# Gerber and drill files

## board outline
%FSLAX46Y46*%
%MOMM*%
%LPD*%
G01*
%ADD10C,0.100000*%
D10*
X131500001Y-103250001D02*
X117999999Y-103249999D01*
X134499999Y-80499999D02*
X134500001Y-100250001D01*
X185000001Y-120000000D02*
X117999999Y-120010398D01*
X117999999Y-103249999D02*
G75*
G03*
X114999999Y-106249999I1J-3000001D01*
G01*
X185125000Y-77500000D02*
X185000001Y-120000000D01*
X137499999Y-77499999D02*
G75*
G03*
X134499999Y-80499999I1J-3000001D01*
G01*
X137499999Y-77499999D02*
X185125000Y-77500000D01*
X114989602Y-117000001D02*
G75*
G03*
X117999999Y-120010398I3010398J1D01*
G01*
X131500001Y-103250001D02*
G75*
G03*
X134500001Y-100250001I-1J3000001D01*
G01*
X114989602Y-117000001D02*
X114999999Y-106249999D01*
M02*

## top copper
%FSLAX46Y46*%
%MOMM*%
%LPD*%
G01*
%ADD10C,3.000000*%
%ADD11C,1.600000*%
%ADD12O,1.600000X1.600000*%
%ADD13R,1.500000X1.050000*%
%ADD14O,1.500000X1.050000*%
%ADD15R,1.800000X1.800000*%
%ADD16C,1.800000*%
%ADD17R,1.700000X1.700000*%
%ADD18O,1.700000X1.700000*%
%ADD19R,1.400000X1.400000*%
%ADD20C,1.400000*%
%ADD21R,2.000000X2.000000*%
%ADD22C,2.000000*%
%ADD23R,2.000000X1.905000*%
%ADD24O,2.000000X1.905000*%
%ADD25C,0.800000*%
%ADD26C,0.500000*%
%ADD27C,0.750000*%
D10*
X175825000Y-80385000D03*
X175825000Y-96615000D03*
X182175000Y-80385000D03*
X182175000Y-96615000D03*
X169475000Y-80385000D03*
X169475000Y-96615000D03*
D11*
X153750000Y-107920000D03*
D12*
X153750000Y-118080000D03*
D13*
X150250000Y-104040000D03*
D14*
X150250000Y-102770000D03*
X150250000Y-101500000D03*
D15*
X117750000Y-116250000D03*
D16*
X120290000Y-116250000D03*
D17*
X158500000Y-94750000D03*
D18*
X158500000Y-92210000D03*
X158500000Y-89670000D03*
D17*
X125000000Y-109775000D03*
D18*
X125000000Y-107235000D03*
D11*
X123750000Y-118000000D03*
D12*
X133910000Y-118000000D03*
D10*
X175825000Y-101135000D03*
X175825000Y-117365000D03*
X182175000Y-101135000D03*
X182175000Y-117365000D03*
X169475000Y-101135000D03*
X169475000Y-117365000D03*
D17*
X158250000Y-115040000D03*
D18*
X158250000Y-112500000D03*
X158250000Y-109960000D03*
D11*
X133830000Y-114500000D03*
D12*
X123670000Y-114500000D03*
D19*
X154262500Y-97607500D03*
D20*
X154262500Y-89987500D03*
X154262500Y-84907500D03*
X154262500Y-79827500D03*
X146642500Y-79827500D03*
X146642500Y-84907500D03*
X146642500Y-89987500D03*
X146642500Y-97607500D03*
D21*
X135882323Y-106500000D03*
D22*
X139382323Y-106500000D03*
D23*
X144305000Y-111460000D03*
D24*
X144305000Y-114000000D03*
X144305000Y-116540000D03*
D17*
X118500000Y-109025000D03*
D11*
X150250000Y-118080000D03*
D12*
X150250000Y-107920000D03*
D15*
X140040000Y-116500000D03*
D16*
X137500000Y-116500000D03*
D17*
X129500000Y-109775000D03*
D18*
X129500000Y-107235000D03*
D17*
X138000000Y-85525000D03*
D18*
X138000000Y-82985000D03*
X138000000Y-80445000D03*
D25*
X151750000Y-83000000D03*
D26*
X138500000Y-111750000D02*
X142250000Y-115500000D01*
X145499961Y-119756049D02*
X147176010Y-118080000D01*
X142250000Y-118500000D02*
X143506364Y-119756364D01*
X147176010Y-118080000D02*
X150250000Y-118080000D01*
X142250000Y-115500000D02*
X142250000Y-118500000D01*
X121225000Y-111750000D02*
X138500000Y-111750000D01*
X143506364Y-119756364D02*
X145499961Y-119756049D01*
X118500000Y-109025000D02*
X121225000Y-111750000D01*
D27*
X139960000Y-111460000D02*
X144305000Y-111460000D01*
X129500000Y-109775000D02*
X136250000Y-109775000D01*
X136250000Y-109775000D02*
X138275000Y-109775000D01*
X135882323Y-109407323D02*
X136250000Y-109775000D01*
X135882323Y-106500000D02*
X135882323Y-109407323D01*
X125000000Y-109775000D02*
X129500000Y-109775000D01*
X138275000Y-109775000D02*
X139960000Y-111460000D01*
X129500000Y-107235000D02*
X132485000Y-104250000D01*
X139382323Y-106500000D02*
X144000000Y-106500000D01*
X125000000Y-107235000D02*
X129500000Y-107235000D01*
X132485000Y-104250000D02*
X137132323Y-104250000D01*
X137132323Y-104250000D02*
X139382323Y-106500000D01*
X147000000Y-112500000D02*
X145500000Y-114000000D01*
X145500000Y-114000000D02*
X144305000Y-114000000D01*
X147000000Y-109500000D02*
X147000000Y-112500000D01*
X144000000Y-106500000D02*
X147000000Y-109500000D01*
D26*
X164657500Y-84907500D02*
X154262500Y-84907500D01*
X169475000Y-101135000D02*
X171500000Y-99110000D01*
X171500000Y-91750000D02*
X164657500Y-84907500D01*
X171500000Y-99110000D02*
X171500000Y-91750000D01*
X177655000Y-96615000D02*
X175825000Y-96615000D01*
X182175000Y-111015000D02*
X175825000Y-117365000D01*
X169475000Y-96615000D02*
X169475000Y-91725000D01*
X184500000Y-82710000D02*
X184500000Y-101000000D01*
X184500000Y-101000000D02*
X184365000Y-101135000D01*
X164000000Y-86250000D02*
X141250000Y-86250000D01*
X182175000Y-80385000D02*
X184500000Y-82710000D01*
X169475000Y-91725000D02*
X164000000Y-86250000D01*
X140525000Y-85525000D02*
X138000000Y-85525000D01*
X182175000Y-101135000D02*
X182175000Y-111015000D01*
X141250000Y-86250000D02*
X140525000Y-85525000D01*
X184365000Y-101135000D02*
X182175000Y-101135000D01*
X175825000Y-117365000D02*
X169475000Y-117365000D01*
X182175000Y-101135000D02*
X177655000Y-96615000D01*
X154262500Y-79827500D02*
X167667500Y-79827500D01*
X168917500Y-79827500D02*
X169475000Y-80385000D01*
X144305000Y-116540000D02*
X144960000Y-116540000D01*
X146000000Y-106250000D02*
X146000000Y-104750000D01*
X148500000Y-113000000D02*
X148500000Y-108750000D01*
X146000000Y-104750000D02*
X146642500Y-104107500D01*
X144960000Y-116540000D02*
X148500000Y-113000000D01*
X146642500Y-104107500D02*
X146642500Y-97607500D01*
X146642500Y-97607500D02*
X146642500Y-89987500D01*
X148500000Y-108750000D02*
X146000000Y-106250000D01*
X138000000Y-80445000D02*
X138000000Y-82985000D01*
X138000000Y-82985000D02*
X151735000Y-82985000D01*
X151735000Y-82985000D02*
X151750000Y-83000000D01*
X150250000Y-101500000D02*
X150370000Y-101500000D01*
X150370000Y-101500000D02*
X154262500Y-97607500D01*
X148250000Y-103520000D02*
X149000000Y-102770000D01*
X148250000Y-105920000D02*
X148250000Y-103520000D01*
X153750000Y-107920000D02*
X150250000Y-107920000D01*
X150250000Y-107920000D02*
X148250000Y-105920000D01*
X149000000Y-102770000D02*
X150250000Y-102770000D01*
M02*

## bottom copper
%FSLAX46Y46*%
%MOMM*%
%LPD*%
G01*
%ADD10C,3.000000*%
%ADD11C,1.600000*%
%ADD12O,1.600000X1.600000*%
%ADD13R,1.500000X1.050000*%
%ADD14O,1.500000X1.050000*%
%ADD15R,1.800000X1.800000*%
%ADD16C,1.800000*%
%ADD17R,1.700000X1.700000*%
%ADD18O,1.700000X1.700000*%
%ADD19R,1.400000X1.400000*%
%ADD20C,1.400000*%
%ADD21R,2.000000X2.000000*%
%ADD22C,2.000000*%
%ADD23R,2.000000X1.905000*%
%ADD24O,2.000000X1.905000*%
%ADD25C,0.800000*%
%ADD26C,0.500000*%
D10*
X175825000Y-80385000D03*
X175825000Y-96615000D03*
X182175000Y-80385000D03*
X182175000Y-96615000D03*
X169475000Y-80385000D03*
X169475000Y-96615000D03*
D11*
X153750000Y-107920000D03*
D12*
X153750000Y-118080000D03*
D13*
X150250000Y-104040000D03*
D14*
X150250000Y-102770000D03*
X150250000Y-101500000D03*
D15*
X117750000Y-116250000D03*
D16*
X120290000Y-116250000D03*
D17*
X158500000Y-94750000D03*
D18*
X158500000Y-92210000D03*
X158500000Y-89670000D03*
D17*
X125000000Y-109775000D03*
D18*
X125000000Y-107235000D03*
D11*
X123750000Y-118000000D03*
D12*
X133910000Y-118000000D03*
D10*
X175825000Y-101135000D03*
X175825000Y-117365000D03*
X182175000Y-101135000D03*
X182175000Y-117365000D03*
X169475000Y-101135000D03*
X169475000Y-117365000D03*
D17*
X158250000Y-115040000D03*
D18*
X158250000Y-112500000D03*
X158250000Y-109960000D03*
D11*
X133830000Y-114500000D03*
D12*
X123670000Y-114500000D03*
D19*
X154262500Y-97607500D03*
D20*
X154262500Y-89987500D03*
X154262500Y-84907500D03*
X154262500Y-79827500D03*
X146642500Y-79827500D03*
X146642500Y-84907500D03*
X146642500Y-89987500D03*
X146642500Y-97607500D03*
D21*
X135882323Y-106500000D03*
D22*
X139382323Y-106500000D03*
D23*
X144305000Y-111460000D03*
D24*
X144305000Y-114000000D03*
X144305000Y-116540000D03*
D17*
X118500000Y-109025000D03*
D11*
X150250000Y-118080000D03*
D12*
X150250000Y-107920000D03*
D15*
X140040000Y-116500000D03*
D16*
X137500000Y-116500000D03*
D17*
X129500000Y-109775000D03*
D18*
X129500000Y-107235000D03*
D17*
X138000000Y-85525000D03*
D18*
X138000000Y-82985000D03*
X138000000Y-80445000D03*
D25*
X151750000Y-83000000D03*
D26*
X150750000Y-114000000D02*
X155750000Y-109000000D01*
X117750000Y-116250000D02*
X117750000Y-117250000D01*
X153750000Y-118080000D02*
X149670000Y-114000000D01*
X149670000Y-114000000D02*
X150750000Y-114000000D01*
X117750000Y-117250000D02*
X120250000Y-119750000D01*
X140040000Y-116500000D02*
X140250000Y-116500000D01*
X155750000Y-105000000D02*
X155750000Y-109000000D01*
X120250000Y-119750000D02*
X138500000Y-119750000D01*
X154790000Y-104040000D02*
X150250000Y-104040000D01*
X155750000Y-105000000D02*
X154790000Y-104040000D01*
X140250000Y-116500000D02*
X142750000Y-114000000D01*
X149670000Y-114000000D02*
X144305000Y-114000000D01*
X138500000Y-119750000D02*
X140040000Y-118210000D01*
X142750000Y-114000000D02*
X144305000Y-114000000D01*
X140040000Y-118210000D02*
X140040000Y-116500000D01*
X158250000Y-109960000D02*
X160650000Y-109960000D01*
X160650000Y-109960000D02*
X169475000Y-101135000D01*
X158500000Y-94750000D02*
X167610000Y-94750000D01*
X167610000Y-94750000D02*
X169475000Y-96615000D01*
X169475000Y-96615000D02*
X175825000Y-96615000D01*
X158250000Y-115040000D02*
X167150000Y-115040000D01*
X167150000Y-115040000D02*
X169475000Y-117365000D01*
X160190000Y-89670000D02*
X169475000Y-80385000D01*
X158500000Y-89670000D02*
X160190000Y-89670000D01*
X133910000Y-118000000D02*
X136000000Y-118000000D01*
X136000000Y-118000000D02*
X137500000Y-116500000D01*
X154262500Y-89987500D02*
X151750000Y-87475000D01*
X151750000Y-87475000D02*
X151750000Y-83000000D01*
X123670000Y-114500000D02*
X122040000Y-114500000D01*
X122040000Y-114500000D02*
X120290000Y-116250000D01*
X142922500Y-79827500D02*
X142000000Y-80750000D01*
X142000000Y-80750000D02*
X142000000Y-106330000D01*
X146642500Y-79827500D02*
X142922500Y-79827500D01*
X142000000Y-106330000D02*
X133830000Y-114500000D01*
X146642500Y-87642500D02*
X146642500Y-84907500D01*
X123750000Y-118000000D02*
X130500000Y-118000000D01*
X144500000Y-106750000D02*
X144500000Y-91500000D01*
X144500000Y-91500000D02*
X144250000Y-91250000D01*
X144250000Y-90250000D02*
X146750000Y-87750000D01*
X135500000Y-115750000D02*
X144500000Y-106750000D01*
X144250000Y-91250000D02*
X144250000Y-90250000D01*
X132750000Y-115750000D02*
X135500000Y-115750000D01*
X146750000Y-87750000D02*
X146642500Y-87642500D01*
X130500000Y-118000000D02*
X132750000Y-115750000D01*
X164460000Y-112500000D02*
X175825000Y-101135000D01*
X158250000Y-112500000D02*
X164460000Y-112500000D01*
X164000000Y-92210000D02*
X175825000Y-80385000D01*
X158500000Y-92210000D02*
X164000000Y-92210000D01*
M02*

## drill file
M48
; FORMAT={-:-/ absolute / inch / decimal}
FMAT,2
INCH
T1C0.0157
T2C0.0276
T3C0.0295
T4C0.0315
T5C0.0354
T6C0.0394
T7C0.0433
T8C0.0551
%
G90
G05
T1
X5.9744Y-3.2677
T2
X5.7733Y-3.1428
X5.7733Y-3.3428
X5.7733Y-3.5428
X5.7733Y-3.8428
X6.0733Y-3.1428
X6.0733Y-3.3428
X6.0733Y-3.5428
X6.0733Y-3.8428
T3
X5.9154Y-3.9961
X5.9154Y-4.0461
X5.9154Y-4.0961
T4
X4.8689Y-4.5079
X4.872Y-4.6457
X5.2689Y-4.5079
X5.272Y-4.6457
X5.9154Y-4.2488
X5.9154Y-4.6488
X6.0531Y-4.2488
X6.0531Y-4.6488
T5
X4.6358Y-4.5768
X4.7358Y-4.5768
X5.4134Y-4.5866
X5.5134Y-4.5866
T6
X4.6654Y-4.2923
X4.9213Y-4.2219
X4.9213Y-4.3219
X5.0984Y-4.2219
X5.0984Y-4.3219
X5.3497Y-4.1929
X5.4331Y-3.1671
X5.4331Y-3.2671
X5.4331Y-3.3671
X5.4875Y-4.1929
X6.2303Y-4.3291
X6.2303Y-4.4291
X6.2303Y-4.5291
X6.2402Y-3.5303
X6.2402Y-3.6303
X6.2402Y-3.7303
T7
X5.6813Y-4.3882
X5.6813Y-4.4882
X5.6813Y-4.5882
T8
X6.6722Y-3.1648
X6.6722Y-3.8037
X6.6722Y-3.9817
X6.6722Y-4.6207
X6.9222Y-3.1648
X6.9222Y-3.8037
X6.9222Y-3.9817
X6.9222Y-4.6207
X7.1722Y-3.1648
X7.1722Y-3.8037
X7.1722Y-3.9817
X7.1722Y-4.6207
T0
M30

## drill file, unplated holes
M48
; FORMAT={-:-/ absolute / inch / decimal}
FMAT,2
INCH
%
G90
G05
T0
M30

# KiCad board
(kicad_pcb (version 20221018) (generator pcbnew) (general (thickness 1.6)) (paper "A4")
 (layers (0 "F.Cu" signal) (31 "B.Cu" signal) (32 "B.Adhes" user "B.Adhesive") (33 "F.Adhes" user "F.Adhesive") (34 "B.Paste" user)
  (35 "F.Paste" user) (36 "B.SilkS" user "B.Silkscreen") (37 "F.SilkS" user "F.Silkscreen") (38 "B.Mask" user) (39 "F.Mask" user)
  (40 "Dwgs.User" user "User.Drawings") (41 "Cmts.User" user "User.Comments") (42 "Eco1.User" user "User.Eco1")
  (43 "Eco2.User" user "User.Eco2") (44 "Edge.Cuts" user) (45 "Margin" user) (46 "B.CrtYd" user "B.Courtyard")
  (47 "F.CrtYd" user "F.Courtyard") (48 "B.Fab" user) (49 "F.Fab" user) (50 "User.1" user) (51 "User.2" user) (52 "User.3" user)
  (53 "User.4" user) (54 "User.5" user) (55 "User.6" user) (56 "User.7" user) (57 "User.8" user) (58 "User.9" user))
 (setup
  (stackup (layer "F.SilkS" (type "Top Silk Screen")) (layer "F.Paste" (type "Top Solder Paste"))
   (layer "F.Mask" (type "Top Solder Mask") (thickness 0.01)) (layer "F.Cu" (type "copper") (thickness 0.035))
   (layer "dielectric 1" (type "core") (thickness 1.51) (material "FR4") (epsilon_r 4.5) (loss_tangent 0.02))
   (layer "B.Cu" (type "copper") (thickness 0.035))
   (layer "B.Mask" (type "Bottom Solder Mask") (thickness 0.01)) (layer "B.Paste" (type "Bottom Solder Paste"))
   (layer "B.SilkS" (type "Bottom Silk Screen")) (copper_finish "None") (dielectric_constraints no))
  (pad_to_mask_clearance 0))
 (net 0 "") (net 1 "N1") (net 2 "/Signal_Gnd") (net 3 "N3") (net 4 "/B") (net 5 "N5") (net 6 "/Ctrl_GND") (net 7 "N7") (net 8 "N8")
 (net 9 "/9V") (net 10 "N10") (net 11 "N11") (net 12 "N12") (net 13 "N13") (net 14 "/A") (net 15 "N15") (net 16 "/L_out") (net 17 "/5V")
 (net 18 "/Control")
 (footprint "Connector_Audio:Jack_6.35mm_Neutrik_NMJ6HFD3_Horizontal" (layer "F.Cu") (at 169.475 80.385)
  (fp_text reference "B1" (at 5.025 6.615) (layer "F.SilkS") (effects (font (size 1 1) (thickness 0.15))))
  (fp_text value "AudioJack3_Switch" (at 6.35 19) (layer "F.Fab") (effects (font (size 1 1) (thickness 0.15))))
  (pad "R" thru_hole circle (at 6.35 0) (size 3 3) (drill 1.4) (layers "*.Cu" "*.Mask") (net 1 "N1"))
  (pad "RN" thru_hole circle (at 6.35 16.23) (size 3 3) (drill 1.4) (layers "*.Cu" "*.Mask") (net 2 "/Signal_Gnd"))
  (pad "S" thru_hole circle (at 12.7 0) (size 3 3) (drill 1.4) (layers "*.Cu" "*.Mask") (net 2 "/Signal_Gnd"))
  (pad "SN" thru_hole circle (at 12.7 16.23) (size 3 3) (drill 1.4) (layers "*.Cu" "*.Mask") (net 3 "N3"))
  (pad "T" thru_hole circle (at 0 0) (size 3 3) (drill 1.4) (layers "*.Cu" "*.Mask") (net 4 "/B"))
  (pad "TN" thru_hole circle (at 0 16.23) (size 3 3) (drill 1.4) (layers "*.Cu" "*.Mask") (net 2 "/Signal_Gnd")))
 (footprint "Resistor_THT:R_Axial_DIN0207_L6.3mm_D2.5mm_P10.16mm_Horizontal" (layer "F.Cu") (at 153.75 107.92 -90)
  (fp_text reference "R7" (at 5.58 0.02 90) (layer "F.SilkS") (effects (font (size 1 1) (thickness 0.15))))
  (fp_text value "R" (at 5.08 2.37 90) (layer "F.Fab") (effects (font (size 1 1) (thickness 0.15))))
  (pad "1" thru_hole circle (at 0 0 270) (size 1.6 1.6) (drill 0.8) (layers "*.Cu" "*.Mask") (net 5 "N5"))
  (pad "2" thru_hole oval (at 10.16 0 270) (size 1.6 1.6) (drill 0.8) (layers "*.Cu" "*.Mask") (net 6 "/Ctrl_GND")))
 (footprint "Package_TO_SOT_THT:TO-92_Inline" (layer "F.Cu") (at 150.25 104.04 90)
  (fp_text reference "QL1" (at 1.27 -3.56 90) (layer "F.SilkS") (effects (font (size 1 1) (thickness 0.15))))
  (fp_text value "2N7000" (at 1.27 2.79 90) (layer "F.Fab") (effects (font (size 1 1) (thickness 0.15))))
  (pad "1" thru_hole rect (at 0 0 90) (size 1.05 1.5) (drill 0.75) (layers "*.Cu" "*.Mask") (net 6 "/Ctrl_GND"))
  (pad "2" thru_hole oval (at 1.27 0 90) (size 1.05 1.5) (drill 0.75) (layers "*.Cu" "*.Mask") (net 5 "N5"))
  (pad "3" thru_hole oval (at 2.54 0 90) (size 1.05 1.5) (drill 0.75) (layers "*.Cu" "*.Mask") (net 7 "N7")))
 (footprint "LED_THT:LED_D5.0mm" (layer "F.Cu") (at 117.75 116.25)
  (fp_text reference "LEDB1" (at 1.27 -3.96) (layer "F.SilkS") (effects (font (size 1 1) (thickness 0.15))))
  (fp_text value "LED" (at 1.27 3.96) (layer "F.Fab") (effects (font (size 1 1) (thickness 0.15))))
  (pad "1" thru_hole rect (at 0 0) (size 1.8 1.8) (drill 0.9) (layers "*.Cu" "*.Mask") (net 6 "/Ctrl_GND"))
  (pad "2" thru_hole circle (at 2.54 0) (size 1.8 1.8) (drill 0.9) (layers "*.Cu" "*.Mask") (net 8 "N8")))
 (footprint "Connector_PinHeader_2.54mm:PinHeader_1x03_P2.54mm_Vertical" (layer "F.Cu") (at 158.5 94.75 180)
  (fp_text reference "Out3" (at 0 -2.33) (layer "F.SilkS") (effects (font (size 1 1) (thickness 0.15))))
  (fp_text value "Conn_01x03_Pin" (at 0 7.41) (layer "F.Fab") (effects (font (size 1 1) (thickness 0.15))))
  (pad "1" thru_hole rect (at 0 0 180) (size 1.7 1.7) (drill 1) (layers "*.Cu" "*.Mask") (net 2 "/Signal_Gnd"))
  (pad "2" thru_hole oval (at 0 2.54 180) (size 1.7 1.7) (drill 1) (layers "*.Cu" "*.Mask") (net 1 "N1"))
  (pad "3" thru_hole oval (at 0 5.08 180) (size 1.7 1.7) (drill 1) (layers "*.Cu" "*.Mask") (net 4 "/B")))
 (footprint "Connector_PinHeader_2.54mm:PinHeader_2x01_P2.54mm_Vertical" (layer "F.Cu") (at 125 109.775 90)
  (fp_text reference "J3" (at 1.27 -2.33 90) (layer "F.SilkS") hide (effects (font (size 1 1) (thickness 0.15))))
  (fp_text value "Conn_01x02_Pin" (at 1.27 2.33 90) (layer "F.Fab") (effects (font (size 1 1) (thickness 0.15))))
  (pad "1" thru_hole rect (at 0 0 90) (size 1.7 1.7) (drill 1) (layers "*.Cu" "*.Mask") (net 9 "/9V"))
  (pad "2" thru_hole oval (at 2.54 0 90) (size 1.7 1.7) (drill 1) (layers "*.Cu" "*.Mask") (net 6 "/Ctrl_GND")))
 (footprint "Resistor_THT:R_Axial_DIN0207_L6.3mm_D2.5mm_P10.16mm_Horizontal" (layer "F.Cu") (at 123.75 118)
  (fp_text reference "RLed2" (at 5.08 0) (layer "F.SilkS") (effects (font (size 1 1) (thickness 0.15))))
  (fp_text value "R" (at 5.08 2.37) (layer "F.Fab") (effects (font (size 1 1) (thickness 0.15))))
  (pad "1" thru_hole circle (at 0 0) (size 1.6 1.6) (drill 0.8) (layers "*.Cu" "*.Mask") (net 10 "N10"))
  (pad "2" thru_hole oval (at 10.16 0) (size 1.6 1.6) (drill 0.8) (layers "*.Cu" "*.Mask") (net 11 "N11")))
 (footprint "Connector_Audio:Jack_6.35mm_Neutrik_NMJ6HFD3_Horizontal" (layer "F.Cu") (at 169.475 101.135)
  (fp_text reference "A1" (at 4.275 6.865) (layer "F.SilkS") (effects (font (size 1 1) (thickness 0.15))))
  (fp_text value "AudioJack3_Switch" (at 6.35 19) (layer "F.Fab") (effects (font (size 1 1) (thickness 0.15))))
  (pad "R" thru_hole circle (at 6.35 0) (size 3 3) (drill 1.4) (layers "*.Cu" "*.Mask") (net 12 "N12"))
  (pad "RN" thru_hole circle (at 6.35 16.23) (size 3 3) (drill 1.4) (layers "*.Cu" "*.Mask") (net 2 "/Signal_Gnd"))
  (pad "S" thru_hole circle (at 12.7 0) (size 3 3) (drill 1.4) (layers "*.Cu" "*.Mask") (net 2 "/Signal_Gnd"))
  (pad "SN" thru_hole circle (at 12.7 16.23) (size 3 3) (drill 1.4) (layers "*.Cu" "*.Mask") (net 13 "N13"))
  (pad "T" thru_hole circle (at 0 0) (size 3 3) (drill 1.4) (layers "*.Cu" "*.Mask") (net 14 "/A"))
  (pad "TN" thru_hole circle (at 0 16.23) (size 3 3) (drill 1.4) (layers "*.Cu" "*.Mask") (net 2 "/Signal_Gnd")))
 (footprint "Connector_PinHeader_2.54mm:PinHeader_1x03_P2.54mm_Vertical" (layer "F.Cu") (at 158.25 115.04 180)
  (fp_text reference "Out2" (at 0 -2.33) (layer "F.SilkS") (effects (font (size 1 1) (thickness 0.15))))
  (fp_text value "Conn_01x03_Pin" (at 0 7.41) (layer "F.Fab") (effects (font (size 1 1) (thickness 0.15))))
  (pad "1" thru_hole rect (at 0 0 180) (size 1.7 1.7) (drill 1) (layers "*.Cu" "*.Mask") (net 2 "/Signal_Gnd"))
  (pad "2" thru_hole oval (at 0 2.54 180) (size 1.7 1.7) (drill 1) (layers "*.Cu" "*.Mask") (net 12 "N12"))
  (pad "3" thru_hole oval (at 0 5.08 180) (size 1.7 1.7) (drill 1) (layers "*.Cu" "*.Mask") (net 14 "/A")))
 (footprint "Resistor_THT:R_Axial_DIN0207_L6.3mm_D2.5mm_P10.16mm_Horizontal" (layer "F.Cu") (at 133.83 114.5 180)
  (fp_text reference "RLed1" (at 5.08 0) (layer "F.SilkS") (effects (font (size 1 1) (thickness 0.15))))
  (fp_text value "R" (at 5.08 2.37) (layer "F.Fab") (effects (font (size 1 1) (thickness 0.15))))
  (pad "1" thru_hole circle (at 0 0 180) (size 1.6 1.6) (drill 0.8) (layers "*.Cu" "*.Mask") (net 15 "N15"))
  (pad "2" thru_hole oval (at 10.16 0 180) (size 1.6 1.6) (drill 0.8) (layers "*.Cu" "*.Mask") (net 8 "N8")))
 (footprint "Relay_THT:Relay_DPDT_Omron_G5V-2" (layer "F.Cu") (at 154.2625 97.6075 180)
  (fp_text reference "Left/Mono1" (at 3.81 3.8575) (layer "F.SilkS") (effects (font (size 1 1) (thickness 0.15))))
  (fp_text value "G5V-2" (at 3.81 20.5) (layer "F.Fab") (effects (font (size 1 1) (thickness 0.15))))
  (pad "1" thru_hole rect (at 0 0 180) (size 1.4 1.4) (drill 0.7) (layers "*.Cu" "*.Mask") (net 7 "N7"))
  (pad "4" thru_hole circle (at 0 7.62 180) (size 1.4 1.4) (drill 0.7) (layers "*.Cu" "*.Mask") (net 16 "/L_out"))
  (pad "6" thru_hole circle (at 0 12.7 180) (size 1.4 1.4) (drill 0.7) (layers "*.Cu" "*.Mask") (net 14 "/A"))
  (pad "8" thru_hole circle (at 0 17.78 180) (size 1.4 1.4) (drill 0.7) (layers "*.Cu" "*.Mask") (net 4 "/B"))
  (pad "9" thru_hole circle (at 7.62 17.78 180) (size 1.4 1.4) (drill 0.7) (layers "*.Cu" "*.Mask") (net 15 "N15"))
  (pad "11" thru_hole circle (at 7.62 12.7 180) (size 1.4 1.4) (drill 0.7) (layers "*.Cu" "*.Mask") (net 10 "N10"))
  (pad "13" thru_hole circle (at 7.62 7.62 180) (size 1.4 1.4) (drill 0.7) (layers "*.Cu" "*.Mask") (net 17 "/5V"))
  (pad "16" thru_hole circle (at 7.62 0 180) (size 1.4 1.4) (drill 0.7) (layers "*.Cu" "*.Mask") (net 17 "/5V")))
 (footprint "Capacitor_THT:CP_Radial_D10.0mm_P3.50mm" (layer "F.Cu") (at 135.882323 106.5)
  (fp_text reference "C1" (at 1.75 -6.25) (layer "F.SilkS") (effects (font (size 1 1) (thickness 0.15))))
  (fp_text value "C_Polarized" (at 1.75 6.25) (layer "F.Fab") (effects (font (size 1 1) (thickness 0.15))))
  (pad "1" thru_hole rect (at 0 0) (size 2 2) (drill 1) (layers "*.Cu" "*.Mask") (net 9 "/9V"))
  (pad "2" thru_hole circle (at 3.5 0) (size 2 2) (drill 1) (layers "*.Cu" "*.Mask") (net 6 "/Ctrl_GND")))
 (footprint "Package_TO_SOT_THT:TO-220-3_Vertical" (layer "F.Cu") (at 144.305 111.46 -90)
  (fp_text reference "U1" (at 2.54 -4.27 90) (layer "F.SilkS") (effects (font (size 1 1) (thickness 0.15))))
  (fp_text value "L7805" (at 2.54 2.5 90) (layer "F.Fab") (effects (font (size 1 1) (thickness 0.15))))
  (pad "1" thru_hole rect (at 0 0 270) (size 1.905 2) (drill 1.1) (layers "*.Cu" "*.Mask") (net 9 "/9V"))
  (pad "2" thru_hole oval (at 2.54 0 270) (size 1.905 2) (drill 1.1) (layers "*.Cu" "*.Mask") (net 6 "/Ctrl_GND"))
  (pad "3" thru_hole oval (at 5.08 0 270) (size 1.905 2) (drill 1.1) (layers "*.Cu" "*.Mask") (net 17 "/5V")))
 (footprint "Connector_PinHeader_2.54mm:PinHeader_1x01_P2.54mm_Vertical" (layer "F.Cu") (at 118.5 109.025 90)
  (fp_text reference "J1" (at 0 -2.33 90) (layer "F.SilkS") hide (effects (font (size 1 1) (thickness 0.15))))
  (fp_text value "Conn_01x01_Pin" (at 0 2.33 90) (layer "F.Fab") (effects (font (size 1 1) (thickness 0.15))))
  (pad "1" thru_hole rect (at 0 0 90) (size 1.7 1.7) (drill 1) (layers "*.Cu" "*.Mask") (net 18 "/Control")))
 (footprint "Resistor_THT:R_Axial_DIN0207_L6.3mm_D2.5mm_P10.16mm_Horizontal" (layer "F.Cu") (at 150.25 118.08 90)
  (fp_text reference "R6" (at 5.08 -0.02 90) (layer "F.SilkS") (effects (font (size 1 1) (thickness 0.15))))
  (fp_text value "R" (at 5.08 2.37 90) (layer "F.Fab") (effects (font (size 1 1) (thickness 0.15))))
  (pad "1" thru_hole circle (at 0 0 90) (size 1.6 1.6) (drill 0.8) (layers "*.Cu" "*.Mask") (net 18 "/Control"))
  (pad "2" thru_hole oval (at 10.16 0 90) (size 1.6 1.6) (drill 0.8) (layers "*.Cu" "*.Mask") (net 5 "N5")))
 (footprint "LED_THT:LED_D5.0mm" (layer "F.Cu") (at 140.04 116.5 180)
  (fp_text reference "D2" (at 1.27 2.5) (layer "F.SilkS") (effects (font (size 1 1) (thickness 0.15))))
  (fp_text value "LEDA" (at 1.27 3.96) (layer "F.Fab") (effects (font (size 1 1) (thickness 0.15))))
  (pad "1" thru_hole rect (at 0 0 180) (size 1.8 1.8) (drill 0.9) (layers "*.Cu" "*.Mask") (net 6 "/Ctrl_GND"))
  (pad "2" thru_hole circle (at 2.54 0 180) (size 1.8 1.8) (drill 0.9) (layers "*.Cu" "*.Mask") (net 11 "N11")))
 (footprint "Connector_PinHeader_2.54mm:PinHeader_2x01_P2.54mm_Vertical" (layer "F.Cu") (at 129.5 109.775 90)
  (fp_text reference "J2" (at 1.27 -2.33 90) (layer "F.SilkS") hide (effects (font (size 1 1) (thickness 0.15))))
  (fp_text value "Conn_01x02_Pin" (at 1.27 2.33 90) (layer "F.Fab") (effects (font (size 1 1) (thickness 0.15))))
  (pad "1" thru_hole rect (at 0 0 90) (size 1.7 1.7) (drill 1) (layers "*.Cu" "*.Mask") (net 9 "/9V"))
  (pad "2" thru_hole oval (at 2.54 0 90) (size 1.7 1.7) (drill 1) (layers "*.Cu" "*.Mask") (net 6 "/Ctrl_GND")))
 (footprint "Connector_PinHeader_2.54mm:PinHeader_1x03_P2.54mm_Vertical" (layer "F.Cu") (at 138 85.525 180)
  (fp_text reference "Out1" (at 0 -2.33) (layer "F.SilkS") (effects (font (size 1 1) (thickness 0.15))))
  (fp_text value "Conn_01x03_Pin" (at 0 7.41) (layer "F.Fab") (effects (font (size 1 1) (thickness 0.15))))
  (pad "1" thru_hole rect (at 0 0 180) (size 1.7 1.7) (drill 1) (layers "*.Cu" "*.Mask") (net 2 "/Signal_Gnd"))
  (pad "2" thru_hole oval (at 0 2.54 180) (size 1.7 1.7) (drill 1) (layers "*.Cu" "*.Mask") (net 16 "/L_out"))
  (pad "3" thru_hole oval (at 0 5.08 180) (size 1.7 1.7) (drill 1) (layers "*.Cu" "*.Mask") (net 16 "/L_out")))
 (gr_line (start 131.500001 103.250001) (end 117.999999 103.249999) (stroke (width 0.1) (type default)) (layer "Edge.Cuts"))
 (gr_line (start 134.499999 80.499999) (end 134.500001 100.250001) (stroke (width 0.1) (type default)) (layer "Edge.Cuts"))
 (gr_line (start 185.000001 120) (end 117.999999 120.010398) (stroke (width 0.1) (type default)) (layer "Edge.Cuts"))
 (gr_arc (start 114.999999 106.249999) (mid 115.878679 104.128679) (end 117.999999 103.249999) (stroke (width 0.1) (type default))
  (layer "Edge.Cuts"))
 (gr_line (start 185.125 77.5) (end 185.000001 120) (stroke (width 0.1) (type default)) (layer "Edge.Cuts"))
 (gr_arc (start 134.499999 80.499999) (mid 135.378679 78.378679) (end 137.499999 77.499999) (stroke (width 0.1) (type default))
  (layer "Edge.Cuts"))
 (gr_line (start 137.499999 77.499999) (end 185.125 77.5) (stroke (width 0.1) (type default)) (layer "Edge.Cuts"))
 (gr_arc (start 117.999999 120.010398) (mid 115.871327 119.128673) (end 114.989602 117.000001) (stroke (width 0.1) (type default))
  (layer "Edge.Cuts"))
 (gr_arc (start 134.500001 100.250001) (mid 133.621321 102.371321) (end 131.500001 103.250001) (stroke (width 0.1) (type default))
  (layer "Edge.Cuts"))
 (gr_line (start 114.989602 117.000001) (end 114.999999 106.249999) (stroke (width 0.1) (type default)) (layer "Edge.Cuts"))
 (segment (start 138.5 111.75) (end 142.25 115.5) (width 0.5) (layer "F.Cu") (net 18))
 (segment (start 145.499961 119.756049) (end 147.17601 118.08) (width 0.5) (layer "F.Cu") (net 18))
 (segment (start 142.25 118.5) (end 143.506364 119.756364) (width 0.5) (layer "F.Cu") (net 18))
 (segment (start 147.17601 118.08) (end 150.25 118.08) (width 0.5) (layer "F.Cu") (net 18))
 (segment (start 142.25 115.5) (end 142.25 118.5) (width 0.5) (layer "F.Cu") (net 18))
 (segment (start 121.225 111.75) (end 138.5 111.75) (width 0.5) (layer "F.Cu") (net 18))
 (segment (start 143.506364 119.756364) (end 145.499961 119.756049) (width 0.5) (layer "F.Cu") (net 18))
 (segment (start 118.5 109.025) (end 121.225 111.75) (width 0.5) (layer "F.Cu") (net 18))
 (segment (start 139.96 111.46) (end 144.305 111.46) (width 0.75) (layer "F.Cu") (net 9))
 (segment (start 129.5 109.775) (end 136.25 109.775) (width 0.75) (layer "F.Cu") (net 9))
 (segment (start 136.25 109.775) (end 138.275 109.775) (width 0.75) (layer "F.Cu") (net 9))
 (segment (start 135.882323 109.407323) (end 136.25 109.775) (width 0.75) (layer "F.Cu") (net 9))
 (segment (start 135.882323 106.5) (end 135.882323 109.407323) (width 0.75) (layer "F.Cu") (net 9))
 (segment (start 125 109.775) (end 129.5 109.775) (width 0.75) (layer "F.Cu") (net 9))
 (segment (start 138.275 109.775) (end 139.96 111.46) (width 0.75) (layer "F.Cu") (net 9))
 (segment (start 129.5 107.235) (end 132.485 104.25) (width 0.75) (layer "F.Cu") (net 6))
 (segment (start 139.382323 106.5) (end 144 106.5) (width 0.75) (layer "F.Cu") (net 6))
 (segment (start 125 107.235) (end 129.5 107.235) (width 0.75) (layer "F.Cu") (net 6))
 (segment (start 132.485 104.25) (end 137.132323 104.25) (width 0.75) (layer "F.Cu") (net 6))
 (segment (start 137.132323 104.25) (end 139.382323 106.5) (width 0.75) (layer "F.Cu") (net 6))
 (segment (start 147 112.5) (end 145.5 114) (width 0.75) (layer "F.Cu") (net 6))
 (segment (start 145.5 114) (end 144.305 114) (width 0.75) (layer "F.Cu") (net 6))
 (segment (start 147 109.5) (end 147 112.5) (width 0.75) (layer "F.Cu") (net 6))
 (segment (start 144 106.5) (end 147 109.5) (width 0.75) (layer "F.Cu") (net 6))
 (segment (start 150.75 114) (end 155.75 109) (width 0.5) (layer "B.Cu") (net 6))
 (segment (start 117.75 116.25) (end 117.75 117.25) (width 0.5) (layer "B.Cu") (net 6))
 (segment (start 153.75 118.08) (end 149.67 114) (width 0.5) (layer "B.Cu") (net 6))
 (segment (start 149.67 114) (end 150.75 114) (width 0.5) (layer "B.Cu") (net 6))
 (segment (start 117.75 117.25) (end 120.25 119.75) (width 0.5) (layer "B.Cu") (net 6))
 (segment (start 140.04 116.5) (end 140.25 116.5) (width 0.5) (layer "B.Cu") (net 6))
 (segment (start 155.75 105) (end 155.75 109) (width 0.5) (layer "B.Cu") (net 6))
 (segment (start 120.25 119.75) (end 138.5 119.75) (width 0.5) (layer "B.Cu") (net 6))
 (segment (start 154.79 104.04) (end 150.25 104.04) (width 0.5) (layer "B.Cu") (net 6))
 (segment (start 155.75 105) (end 154.79 104.04) (width 0.5) (layer "B.Cu") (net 6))
 (segment (start 140.25 116.5) (end 142.75 114) (width 0.5) (layer "B.Cu") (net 6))
 (segment (start 149.67 114) (end 144.305 114) (width 0.5) (layer "B.Cu") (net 6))
 (segment (start 138.5 119.75) (end 140.04 118.21) (width 0.5) (layer "B.Cu") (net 6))
 (segment (start 142.75 114) (end 144.305 114) (width 0.5) (layer "B.Cu") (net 6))
 (segment (start 140.04 118.21) (end 140.04 116.5) (width 0.5) (layer "B.Cu") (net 6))
 (segment (start 164.6575 84.9075) (end 154.2625 84.9075) (width 0.5) (layer "F.Cu") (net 14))
 (segment (start 169.475 101.135) (end 171.5 99.11) (width 0.5) (layer "F.Cu") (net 14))
 (segment (start 171.5 91.75) (end 164.6575 84.9075) (width 0.5) (layer "F.Cu") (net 14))
 (segment (start 171.5 99.11) (end 171.5 91.75) (width 0.5) (layer "F.Cu") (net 14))
 (segment (start 158.25 109.96) (end 160.65 109.96) (width 0.5) (layer "B.Cu") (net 14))
 (segment (start 160.65 109.96) (end 169.475 101.135) (width 0.5) (layer "B.Cu") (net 14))
 (segment (start 177.655 96.615) (end 175.825 96.615) (width 0.5) (layer "F.Cu") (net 2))
 (segment (start 182.175 111.015) (end 175.825 117.365) (width 0.5) (layer "F.Cu") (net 2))
 (segment (start 169.475 96.615) (end 169.475 91.725) (width 0.5) (layer "F.Cu") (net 2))
 (segment (start 184.5 82.71) (end 184.5 101) (width 0.5) (layer "F.Cu") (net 2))
 (segment (start 184.5 101) (end 184.365 101.135) (width 0.5) (layer "F.Cu") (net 2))
 (segment (start 164 86.25) (end 141.25 86.25) (width 0.5) (layer "F.Cu") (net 2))
 (segment (start 182.175 80.385) (end 184.5 82.71) (width 0.5) (layer "F.Cu") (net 2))
 (segment (start 169.475 91.725) (end 164 86.25) (width 0.5) (layer "F.Cu") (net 2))
 (segment (start 140.525 85.525) (end 138 85.525) (width 0.5) (layer "F.Cu") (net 2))
 (segment (start 182.175 101.135) (end 182.175 111.015) (width 0.5) (layer "F.Cu") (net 2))
 (segment (start 141.25 86.25) (end 140.525 85.525) (width 0.5) (layer "F.Cu") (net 2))
 (segment (start 184.365 101.135) (end 182.175 101.135) (width 0.5) (layer "F.Cu") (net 2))
 (segment (start 175.825 117.365) (end 169.475 117.365) (width 0.5) (layer "F.Cu") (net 2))
 (segment (start 182.175 101.135) (end 177.655 96.615) (width 0.5) (layer "F.Cu") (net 2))
 (segment (start 158.5 94.75) (end 167.61 94.75) (width 0.5) (layer "B.Cu") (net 2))
 (segment (start 167.61 94.75) (end 169.475 96.615) (width 0.5) (layer "B.Cu") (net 2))
 (segment (start 169.475 96.615) (end 175.825 96.615) (width 0.5) (layer "B.Cu") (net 2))
 (segment (start 158.25 115.04) (end 167.15 115.04) (width 0.5) (layer "B.Cu") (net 2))
 (segment (start 167.15 115.04) (end 169.475 117.365) (width 0.5) (layer "B.Cu") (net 2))
 (segment (start 154.2625 79.8275) (end 167.6675 79.8275) (width 0.5) (layer "F.Cu") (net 4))
 (segment (start 168.9175 79.8275) (end 169.475 80.385) (width 0.5) (layer "F.Cu") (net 4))
 (segment (start 160.19 89.67) (end 169.475 80.385) (width 0.5) (layer "B.Cu") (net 4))
 (segment (start 158.5 89.67) (end 160.19 89.67) (width 0.5) (layer "B.Cu") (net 4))
 (segment (start 133.91 118) (end 136 118) (width 0.5) (layer "B.Cu") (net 11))
 (segment (start 136 118) (end 137.5 116.5) (width 0.5) (layer "B.Cu") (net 11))
 (segment (start 144.305 116.54) (end 144.96 116.54) (width 0.5) (layer "F.Cu") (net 17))
 (segment (start 146 106.25) (end 146 104.75) (width 0.5) (layer "F.Cu") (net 17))
 (segment (start 148.5 113) (end 148.5 108.75) (width 0.5) (layer "F.Cu") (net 17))
 (segment (start 146 104.75) (end 146.6425 104.1075) (width 0.5) (layer "F.Cu") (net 17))
 (segment (start 144.96 116.54) (end 148.5 113) (width 0.5) (layer "F.Cu") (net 17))
 (segment (start 146.6425 104.1075) (end 146.6425 97.6075) (width 0.5) (layer "F.Cu") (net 17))
 (segment (start 146.6425 97.6075) (end 146.6425 89.9875) (width 0.5) (layer "F.Cu") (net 17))
 (segment (start 148.5 108.75) (end 146 106.25) (width 0.5) (layer "F.Cu") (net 17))
 (segment (start 138 80.445) (end 138 82.985) (width 0.5) (layer "F.Cu") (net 16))
 (segment (start 138 82.985) (end 151.735 82.985) (width 0.5) (layer "F.Cu") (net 16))
 (segment (start 151.735 82.985) (end 151.75 83) (width 0.5) (layer "F.Cu") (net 16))
 (via (at 151.75 83) (size 0.8) (drill 0.4) (layers "F.Cu" "B.Cu") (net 16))
 (segment (start 154.2625 89.9875) (end 151.75 87.475) (width 0.5) (layer "B.Cu") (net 16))
 (segment (start 151.75 87.475) (end 151.75 83) (width 0.5) (layer "B.Cu") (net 16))
 (segment (start 123.67 114.5) (end 122.04 114.5) (width 0.5) (layer "B.Cu") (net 8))
 (segment (start 122.04 114.5) (end 120.29 116.25) (width 0.5) (layer "B.Cu") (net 8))
 (segment (start 142.9225 79.8275) (end 142 80.75) (width 0.5) (layer "B.Cu") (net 15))
 (segment (start 142 80.75) (end 142 106.33) (width 0.5) (layer "B.Cu") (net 15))
 (segment (start 146.6425 79.8275) (end 142.9225 79.8275) (width 0.5) (layer "B.Cu") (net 15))
 (segment (start 142 106.33) (end 133.83 114.5) (width 0.5) (layer "B.Cu") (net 15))
 (segment (start 146.6425 87.6425) (end 146.6425 84.9075) (width 0.5) (layer "B.Cu") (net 10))
 (segment (start 123.75 118) (end 130.5 118) (width 0.5) (layer "B.Cu") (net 10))
 (segment (start 144.5 106.75) (end 144.5 91.5) (width 0.5) (layer "B.Cu") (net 10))
 (segment (start 144.5 91.5) (end 144.25 91.25) (width 0.5) (layer "B.Cu") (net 10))
 (segment (start 144.25 90.25) (end 146.75 87.75) (width 0.5) (layer "B.Cu") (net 10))
 (segment (start 135.5 115.75) (end 144.5 106.75) (width 0.5) (layer "B.Cu") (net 10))
 (segment (start 144.25 91.25) (end 144.25 90.25) (width 0.5) (layer "B.Cu") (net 10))
 (segment (start 132.75 115.75) (end 135.5 115.75) (width 0.5) (layer "B.Cu") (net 10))
 (segment (start 146.75 87.75) (end 146.6425 87.6425) (width 0.5) (layer "B.Cu") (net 10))
 (segment (start 130.5 118) (end 132.75 115.75) (width 0.5) (layer "B.Cu") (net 10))
 (segment (start 164.46 112.5) (end 175.825 101.135) (width 0.5) (layer "B.Cu") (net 12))
 (segment (start 158.25 112.5) (end 164.46 112.5) (width 0.5) (layer "B.Cu") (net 12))
 (segment (start 164 92.21) (end 175.825 80.385) (width 0.5) (layer "B.Cu") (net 1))
 (segment (start 158.5 92.21) (end 164 92.21) (width 0.5) (layer "B.Cu") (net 1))
 (segment (start 150.25 101.5) (end 150.37 101.5) (width 0.5) (layer "F.Cu") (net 7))
 (segment (start 150.37 101.5) (end 154.2625 97.6075) (width 0.5) (layer "F.Cu") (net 7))
 (segment (start 148.25 103.52) (end 149 102.77) (width 0.5) (layer "F.Cu") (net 5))
 (segment (start 148.25 105.92) (end 148.25 103.52) (width 0.5) (layer "F.Cu") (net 5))
 (segment (start 153.75 107.92) (end 150.25 107.92) (width 0.5) (layer "F.Cu") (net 5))
 (segment (start 150.25 107.92) (end 148.25 105.92) (width 0.5) (layer "F.Cu") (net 5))
 (segment (start 149 102.77) (end 150.25 102.77) (width 0.5) (layer "F.Cu") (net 5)))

